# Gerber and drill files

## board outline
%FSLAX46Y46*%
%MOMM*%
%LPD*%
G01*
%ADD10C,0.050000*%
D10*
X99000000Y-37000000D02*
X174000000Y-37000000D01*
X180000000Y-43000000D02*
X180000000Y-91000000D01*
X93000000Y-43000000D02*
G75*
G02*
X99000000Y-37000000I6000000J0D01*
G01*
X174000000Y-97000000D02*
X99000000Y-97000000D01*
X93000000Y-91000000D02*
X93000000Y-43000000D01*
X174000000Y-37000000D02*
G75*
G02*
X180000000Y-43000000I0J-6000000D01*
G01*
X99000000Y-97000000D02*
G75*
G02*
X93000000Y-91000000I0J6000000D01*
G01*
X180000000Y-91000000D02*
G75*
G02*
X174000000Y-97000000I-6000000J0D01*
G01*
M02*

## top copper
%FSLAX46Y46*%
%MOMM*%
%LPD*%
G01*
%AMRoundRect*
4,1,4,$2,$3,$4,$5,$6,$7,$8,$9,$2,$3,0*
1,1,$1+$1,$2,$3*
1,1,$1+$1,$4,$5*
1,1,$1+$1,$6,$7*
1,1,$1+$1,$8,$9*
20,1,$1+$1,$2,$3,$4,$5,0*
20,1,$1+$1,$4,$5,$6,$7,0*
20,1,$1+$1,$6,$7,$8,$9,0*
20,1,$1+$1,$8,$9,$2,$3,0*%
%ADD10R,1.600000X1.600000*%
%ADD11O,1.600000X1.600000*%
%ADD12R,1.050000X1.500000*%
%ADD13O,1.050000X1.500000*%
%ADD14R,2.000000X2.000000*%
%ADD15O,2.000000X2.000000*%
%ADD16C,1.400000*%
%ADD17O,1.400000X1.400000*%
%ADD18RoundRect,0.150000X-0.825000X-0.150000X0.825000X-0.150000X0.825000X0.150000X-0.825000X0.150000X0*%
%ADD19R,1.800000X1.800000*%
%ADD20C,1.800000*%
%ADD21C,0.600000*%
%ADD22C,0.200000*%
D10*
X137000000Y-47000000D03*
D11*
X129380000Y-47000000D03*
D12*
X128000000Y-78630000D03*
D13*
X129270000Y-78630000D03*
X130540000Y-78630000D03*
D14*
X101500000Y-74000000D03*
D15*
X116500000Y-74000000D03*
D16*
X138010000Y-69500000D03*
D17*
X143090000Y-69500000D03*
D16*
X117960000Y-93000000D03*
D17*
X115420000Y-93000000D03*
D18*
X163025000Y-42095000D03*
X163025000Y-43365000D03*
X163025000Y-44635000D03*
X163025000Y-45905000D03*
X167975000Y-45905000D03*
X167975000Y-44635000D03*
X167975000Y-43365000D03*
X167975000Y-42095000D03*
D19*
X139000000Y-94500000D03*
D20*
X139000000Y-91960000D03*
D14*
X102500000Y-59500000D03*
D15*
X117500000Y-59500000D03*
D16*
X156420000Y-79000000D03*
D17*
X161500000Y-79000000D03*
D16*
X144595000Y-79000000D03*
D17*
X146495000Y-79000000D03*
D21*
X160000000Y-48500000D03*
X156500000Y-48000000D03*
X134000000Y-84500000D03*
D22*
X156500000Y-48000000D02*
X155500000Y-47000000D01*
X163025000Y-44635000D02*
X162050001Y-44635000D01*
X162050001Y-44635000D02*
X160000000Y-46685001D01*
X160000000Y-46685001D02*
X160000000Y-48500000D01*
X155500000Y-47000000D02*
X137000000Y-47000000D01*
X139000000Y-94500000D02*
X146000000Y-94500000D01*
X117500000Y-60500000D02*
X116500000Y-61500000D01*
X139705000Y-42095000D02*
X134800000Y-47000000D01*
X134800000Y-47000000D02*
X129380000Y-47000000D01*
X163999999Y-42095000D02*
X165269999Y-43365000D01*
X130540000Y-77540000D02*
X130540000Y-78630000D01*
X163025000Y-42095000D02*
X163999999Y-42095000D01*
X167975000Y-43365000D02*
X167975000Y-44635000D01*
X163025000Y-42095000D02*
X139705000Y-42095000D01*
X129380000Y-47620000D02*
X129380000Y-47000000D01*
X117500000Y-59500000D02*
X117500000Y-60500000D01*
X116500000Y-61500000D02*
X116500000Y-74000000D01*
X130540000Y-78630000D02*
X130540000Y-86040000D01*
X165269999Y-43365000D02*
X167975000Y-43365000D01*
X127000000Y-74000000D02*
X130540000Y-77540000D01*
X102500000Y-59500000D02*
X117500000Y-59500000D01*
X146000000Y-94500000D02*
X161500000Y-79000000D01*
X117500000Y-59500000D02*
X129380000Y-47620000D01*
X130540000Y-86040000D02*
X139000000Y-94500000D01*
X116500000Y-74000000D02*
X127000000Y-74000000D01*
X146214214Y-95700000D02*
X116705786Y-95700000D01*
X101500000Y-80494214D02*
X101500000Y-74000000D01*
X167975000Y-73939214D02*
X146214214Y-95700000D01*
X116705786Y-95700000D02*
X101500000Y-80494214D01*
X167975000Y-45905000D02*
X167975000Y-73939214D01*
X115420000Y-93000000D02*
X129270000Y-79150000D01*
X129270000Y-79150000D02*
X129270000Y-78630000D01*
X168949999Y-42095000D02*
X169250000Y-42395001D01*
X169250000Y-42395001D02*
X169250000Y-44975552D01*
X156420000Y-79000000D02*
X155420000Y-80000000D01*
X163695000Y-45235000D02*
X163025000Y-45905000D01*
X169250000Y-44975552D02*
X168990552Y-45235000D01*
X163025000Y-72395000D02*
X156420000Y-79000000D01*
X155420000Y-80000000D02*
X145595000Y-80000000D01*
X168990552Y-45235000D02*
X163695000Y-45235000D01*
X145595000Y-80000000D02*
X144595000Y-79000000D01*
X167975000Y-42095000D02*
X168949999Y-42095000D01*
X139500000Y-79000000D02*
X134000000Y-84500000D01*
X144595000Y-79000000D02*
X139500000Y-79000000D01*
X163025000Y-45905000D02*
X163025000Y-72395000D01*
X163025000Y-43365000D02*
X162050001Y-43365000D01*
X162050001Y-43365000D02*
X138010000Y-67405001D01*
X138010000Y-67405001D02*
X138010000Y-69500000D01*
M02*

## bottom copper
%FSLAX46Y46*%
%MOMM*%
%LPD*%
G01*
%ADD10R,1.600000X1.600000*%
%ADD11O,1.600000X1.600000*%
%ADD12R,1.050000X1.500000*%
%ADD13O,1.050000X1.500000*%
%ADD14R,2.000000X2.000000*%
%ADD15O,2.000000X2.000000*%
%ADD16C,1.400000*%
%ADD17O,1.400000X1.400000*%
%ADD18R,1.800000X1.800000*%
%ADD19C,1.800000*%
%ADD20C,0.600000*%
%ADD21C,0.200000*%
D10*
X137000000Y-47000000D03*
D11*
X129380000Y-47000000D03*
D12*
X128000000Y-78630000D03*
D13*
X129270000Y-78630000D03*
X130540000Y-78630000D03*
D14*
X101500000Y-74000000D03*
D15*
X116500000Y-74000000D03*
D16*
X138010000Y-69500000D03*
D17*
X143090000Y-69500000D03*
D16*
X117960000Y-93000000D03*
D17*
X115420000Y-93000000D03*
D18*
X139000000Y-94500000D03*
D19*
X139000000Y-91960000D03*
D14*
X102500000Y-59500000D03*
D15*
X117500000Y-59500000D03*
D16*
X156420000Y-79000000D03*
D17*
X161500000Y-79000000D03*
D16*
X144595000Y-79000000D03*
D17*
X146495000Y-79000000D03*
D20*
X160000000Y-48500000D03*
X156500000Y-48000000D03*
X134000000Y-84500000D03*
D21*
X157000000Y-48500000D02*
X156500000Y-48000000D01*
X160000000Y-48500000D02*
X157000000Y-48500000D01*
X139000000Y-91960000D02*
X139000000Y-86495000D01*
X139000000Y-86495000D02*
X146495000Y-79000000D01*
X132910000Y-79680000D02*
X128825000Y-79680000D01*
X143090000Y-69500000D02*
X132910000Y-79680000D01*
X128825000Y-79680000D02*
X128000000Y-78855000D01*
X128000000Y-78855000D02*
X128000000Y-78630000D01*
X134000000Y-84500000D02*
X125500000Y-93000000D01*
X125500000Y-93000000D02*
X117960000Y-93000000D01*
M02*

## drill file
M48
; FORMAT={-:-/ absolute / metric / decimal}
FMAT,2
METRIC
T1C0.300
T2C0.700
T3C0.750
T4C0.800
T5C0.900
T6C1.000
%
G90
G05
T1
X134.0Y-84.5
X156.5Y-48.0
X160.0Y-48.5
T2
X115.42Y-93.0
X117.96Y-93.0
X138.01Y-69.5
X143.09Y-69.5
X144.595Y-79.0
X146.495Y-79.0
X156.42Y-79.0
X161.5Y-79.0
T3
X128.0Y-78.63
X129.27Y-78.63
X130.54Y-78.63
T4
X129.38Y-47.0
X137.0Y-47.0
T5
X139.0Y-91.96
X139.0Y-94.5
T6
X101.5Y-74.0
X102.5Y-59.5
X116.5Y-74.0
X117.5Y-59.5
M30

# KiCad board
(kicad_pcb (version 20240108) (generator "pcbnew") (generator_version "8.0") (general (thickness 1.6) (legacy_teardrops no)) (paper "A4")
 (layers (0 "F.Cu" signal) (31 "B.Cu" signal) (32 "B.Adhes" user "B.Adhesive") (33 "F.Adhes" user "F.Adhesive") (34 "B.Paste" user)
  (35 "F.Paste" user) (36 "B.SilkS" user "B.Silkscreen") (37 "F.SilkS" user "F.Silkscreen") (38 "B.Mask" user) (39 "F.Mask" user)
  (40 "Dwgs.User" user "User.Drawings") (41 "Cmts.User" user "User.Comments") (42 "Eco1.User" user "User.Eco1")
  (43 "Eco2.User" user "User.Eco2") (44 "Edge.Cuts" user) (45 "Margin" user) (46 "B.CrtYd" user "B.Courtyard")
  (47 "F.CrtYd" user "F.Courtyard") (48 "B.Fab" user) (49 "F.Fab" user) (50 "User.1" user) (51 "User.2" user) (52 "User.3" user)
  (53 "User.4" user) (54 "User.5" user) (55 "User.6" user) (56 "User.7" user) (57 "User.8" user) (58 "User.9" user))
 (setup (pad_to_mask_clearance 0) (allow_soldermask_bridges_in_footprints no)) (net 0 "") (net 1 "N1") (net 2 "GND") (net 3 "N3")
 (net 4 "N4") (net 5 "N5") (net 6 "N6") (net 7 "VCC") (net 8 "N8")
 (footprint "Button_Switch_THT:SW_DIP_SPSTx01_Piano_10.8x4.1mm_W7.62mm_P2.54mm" (layer "F.Cu") (at 137 47 180)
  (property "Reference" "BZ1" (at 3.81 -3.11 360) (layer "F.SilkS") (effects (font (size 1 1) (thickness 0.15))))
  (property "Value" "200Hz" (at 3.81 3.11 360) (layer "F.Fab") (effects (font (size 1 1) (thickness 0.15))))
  (pad "1" thru_hole rect (at 0 0 180) (size 1.6 1.6) (drill 0.8) (layers "*.Cu" "*.Mask") (remove_unused_layers no) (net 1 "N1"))
  (pad "2" thru_hole oval (at 7.62 0 180) (size 1.6 1.6) (drill 0.8) (layers "*.Cu" "*.Mask") (remove_unused_layers no) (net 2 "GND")))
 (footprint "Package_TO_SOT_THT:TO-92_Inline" (layer "F.Cu") (at 128 78.63)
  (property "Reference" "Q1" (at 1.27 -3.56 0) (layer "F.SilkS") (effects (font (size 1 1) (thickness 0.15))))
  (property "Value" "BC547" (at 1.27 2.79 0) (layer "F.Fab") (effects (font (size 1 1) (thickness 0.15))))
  (pad "1" thru_hole rect (at 0 0) (size 1.05 1.5) (drill 0.75) (layers "*.Cu" "*.Mask") (remove_unused_layers no) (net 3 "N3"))
  (pad "2" thru_hole oval (at 1.27 0) (size 1.05 1.5) (drill 0.75) (layers "*.Cu" "*.Mask") (remove_unused_layers no) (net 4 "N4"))
  (pad "3" thru_hole oval (at 2.54 0) (size 1.05 1.5) (drill 0.75) (layers "*.Cu" "*.Mask") (remove_unused_layers no) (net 2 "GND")))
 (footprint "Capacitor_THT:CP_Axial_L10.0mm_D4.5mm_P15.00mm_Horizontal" (layer "F.Cu") (at 101.5 74)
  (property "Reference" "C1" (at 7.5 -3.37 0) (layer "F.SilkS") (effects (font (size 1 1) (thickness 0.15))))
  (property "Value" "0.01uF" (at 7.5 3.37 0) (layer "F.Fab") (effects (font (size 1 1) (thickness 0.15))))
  (pad "1" thru_hole rect (at 0 0) (size 2 2) (drill 1) (layers "*.Cu" "*.Mask") (remove_unused_layers no) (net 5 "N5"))
  (pad "2" thru_hole oval (at 15 0) (size 2 2) (drill 1) (layers "*.Cu" "*.Mask") (remove_unused_layers no) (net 2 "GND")))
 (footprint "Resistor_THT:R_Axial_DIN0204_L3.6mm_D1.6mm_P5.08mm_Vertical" (layer "F.Cu") (at 138.01 69.5)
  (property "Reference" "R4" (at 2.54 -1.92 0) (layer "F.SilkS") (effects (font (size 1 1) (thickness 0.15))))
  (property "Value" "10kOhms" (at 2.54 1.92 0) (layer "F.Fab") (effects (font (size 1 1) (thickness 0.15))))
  (pad "1" thru_hole circle (at 0 0) (size 1.4 1.4) (drill 0.7) (layers "*.Cu" "*.Mask") (remove_unused_layers no) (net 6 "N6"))
  (pad "2" thru_hole oval (at 5.08 0) (size 1.4 1.4) (drill 0.7) (layers "*.Cu" "*.Mask") (remove_unused_layers no) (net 3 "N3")))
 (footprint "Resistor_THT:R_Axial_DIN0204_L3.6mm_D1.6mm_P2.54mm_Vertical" (layer "F.Cu") (at 117.96 93 180)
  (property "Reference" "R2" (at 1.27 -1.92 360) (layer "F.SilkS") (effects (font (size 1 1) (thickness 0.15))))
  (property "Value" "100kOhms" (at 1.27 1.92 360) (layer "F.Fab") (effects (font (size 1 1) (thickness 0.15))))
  (pad "1" thru_hole circle (at 0 0 180) (size 1.4 1.4) (drill 0.7) (layers "*.Cu" "*.Mask") (remove_unused_layers no) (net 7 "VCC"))
  (pad "2" thru_hole oval (at 2.54 0 180) (size 1.4 1.4) (drill 0.7) (layers "*.Cu" "*.Mask") (remove_unused_layers no) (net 4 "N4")))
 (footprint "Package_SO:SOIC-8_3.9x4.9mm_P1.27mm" (layer "F.Cu") (at 165.5 44)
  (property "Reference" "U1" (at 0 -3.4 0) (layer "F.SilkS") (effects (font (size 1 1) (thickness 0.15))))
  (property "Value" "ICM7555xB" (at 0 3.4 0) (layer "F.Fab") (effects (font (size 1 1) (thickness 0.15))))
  (pad "1" smd roundrect (at -2.475 -1.905) (size 1.95 0.6) (layers "F.Cu" "F.Paste" "F.Mask") (roundrect_rratio 0.25) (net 2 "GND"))
  (pad "2" smd roundrect (at -2.475 -0.635) (size 1.95 0.6) (layers "F.Cu" "F.Paste" "F.Mask") (roundrect_rratio 0.25) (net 6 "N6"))
  (pad "3" smd roundrect (at -2.475 0.635) (size 1.95 0.6) (layers "F.Cu" "F.Paste" "F.Mask") (roundrect_rratio 0.25) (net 1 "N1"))
  (pad "4" smd roundrect (at -2.475 1.905) (size 1.95 0.6) (layers "F.Cu" "F.Paste" "F.Mask") (roundrect_rratio 0.25) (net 7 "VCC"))
  (pad "5" smd roundrect (at 2.475 1.905) (size 1.95 0.6) (layers "F.Cu" "F.Paste" "F.Mask") (roundrect_rratio 0.25) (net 5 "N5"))
  (pad "6" smd roundrect (at 2.475 0.635) (size 1.95 0.6) (layers "F.Cu" "F.Paste" "F.Mask") (roundrect_rratio 0.25) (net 2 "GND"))
  (pad "7" smd roundrect (at 2.475 -0.635) (size 1.95 0.6) (layers "F.Cu" "F.Paste" "F.Mask") (roundrect_rratio 0.25) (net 2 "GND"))
  (pad "8" smd roundrect (at 2.475 -1.905) (size 1.95 0.6) (layers "F.Cu" "F.Paste" "F.Mask") (roundrect_rratio 0.25) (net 7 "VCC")))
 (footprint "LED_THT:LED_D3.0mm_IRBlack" (layer "F.Cu") (at 139 94.5 90)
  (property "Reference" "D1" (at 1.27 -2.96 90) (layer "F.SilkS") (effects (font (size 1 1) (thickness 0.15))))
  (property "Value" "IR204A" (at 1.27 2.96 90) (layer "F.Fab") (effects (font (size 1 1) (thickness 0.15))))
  (pad "1" thru_hole rect (at 0 0 90) (size 1.8 1.8) (drill 0.9) (layers "*.Cu" "*.Mask") (remove_unused_layers no) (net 2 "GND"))
  (pad "2" thru_hole circle (at 2.54 0 90) (size 1.8 1.8) (drill 0.9) (layers "*.Cu" "*.Mask") (remove_unused_layers no) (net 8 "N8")))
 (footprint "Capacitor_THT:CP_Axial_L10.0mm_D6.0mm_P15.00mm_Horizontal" (layer "F.Cu") (at 102.5 59.5)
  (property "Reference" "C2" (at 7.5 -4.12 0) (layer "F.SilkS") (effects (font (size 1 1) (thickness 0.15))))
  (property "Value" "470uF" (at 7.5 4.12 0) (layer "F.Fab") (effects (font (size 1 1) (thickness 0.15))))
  (pad "1" thru_hole rect (at 0 0) (size 2 2) (drill 1) (layers "*.Cu" "*.Mask") (remove_unused_layers no) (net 2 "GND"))
  (pad "2" thru_hole oval (at 15 0) (size 2 2) (drill 1) (layers "*.Cu" "*.Mask") (remove_unused_layers no) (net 2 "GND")))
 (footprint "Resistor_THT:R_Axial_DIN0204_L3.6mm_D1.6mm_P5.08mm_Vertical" (layer "F.Cu") (at 156.42 79)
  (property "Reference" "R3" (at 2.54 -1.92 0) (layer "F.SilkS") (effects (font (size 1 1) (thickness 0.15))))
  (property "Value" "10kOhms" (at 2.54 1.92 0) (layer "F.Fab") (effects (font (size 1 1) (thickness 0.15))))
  (pad "1" thru_hole circle (at 0 0) (size 1.4 1.4) (drill 0.7) (layers "*.Cu" "*.Mask") (remove_unused_layers no) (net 7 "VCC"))
  (pad "2" thru_hole oval (at 5.08 0) (size 1.4 1.4) (drill 0.7) (layers "*.Cu" "*.Mask") (remove_unused_layers no) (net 2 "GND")))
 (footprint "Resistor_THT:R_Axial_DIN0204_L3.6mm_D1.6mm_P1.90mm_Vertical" (layer "F.Cu") (at 144.595 79)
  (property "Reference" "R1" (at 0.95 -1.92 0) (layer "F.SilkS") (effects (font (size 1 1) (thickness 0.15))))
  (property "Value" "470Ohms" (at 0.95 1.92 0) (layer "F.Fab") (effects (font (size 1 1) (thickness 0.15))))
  (pad "1" thru_hole circle (at 0 0) (size 1.4 1.4) (drill 0.7) (layers "*.Cu" "*.Mask") (remove_unused_layers no) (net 7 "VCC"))
  (pad "2" thru_hole oval (at 1.9 0) (size 1.4 1.4) (drill 0.7) (layers "*.Cu" "*.Mask") (remove_unused_layers no) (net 8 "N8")))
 (gr_line (start 99 37) (end 174 37) (stroke (width 0.05) (type default)) (layer "Edge.Cuts"))
 (gr_line (start 180 43) (end 180 91) (stroke (width 0.05) (type default)) (layer "Edge.Cuts"))
 (gr_arc (start 93 43) (mid 94.757359 38.757359) (end 99 37) (stroke (width 0.05) (type default)) (layer "Edge.Cuts"))
 (gr_line (start 174 97) (end 99 97) (stroke (width 0.05) (type default)) (layer "Edge.Cuts"))
 (gr_line (start 93 91) (end 93 43) (stroke (width 0.05) (type default)) (layer "Edge.Cuts"))
 (gr_arc (start 174 37) (mid 178.242641 38.757359) (end 180 43) (stroke (width 0.05) (type default)) (layer "Edge.Cuts"))
 (gr_arc (start 99 97) (mid 94.757359 95.242641) (end 93 91) (stroke (width 0.05) (type default)) (layer "Edge.Cuts"))
 (gr_arc (start 180 91) (mid 178.242641 95.242641) (end 174 97) (stroke (width 0.05) (type default)) (layer "Edge.Cuts"))
 (segment (start 156.5 48) (end 155.5 47) (width 0.2) (layer "F.Cu") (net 1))
 (segment (start 163.025 44.635) (end 162.050001 44.635) (width 0.2) (layer "F.Cu") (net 1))
 (segment (start 162.050001 44.635) (end 160 46.685001) (width 0.2) (layer "F.Cu") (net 1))
 (segment (start 160 46.685001) (end 160 48.5) (width 0.2) (layer "F.Cu") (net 1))
 (segment (start 155.5 47) (end 137 47) (width 0.2) (layer "F.Cu") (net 1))
 (via (at 160 48.5) (size 0.6) (drill 0.3) (layers "F.Cu" "B.Cu") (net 1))
 (via (at 156.5 48) (size 0.6) (drill 0.3) (layers "F.Cu" "B.Cu") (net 1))
 (segment (start 157 48.5) (end 156.5 48) (width 0.2) (layer "B.Cu") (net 1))
 (segment (start 160 48.5) (end 157 48.5) (width 0.2) (layer "B.Cu") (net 1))
 (segment (start 139 94.5) (end 146 94.5) (width 0.2) (layer "F.Cu") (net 2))
 (segment (start 117.5 60.5) (end 116.5 61.5) (width 0.2) (layer "F.Cu") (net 2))
 (segment (start 139.705 42.095) (end 134.8 47) (width 0.2) (layer "F.Cu") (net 2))
 (segment (start 134.8 47) (end 129.38 47) (width 0.2) (layer "F.Cu") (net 2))
 (segment (start 163.999999 42.095) (end 165.269999 43.365) (width 0.2) (layer "F.Cu") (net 2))
 (segment (start 130.54 77.54) (end 130.54 78.63) (width 0.2) (layer "F.Cu") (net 2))
 (segment (start 163.025 42.095) (end 163.999999 42.095) (width 0.2) (layer "F.Cu") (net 2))
 (segment (start 167.975 43.365) (end 167.975 44.635) (width 0.2) (layer "F.Cu") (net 2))
 (segment (start 163.025 42.095) (end 139.705 42.095) (width 0.2) (layer "F.Cu") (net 2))
 (segment (start 129.38 47.62) (end 129.38 47) (width 0.2) (layer "F.Cu") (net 2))
 (segment (start 117.5 59.5) (end 117.5 60.5) (width 0.2) (layer "F.Cu") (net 2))
 (segment (start 116.5 61.5) (end 116.5 74) (width 0.2) (layer "F.Cu") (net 2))
 (segment (start 130.54 78.63) (end 130.54 86.04) (width 0.2) (layer "F.Cu") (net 2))
 (segment (start 165.269999 43.365) (end 167.975 43.365) (width 0.2) (layer "F.Cu") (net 2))
 (segment (start 127 74) (end 130.54 77.54) (width 0.2) (layer "F.Cu") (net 2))
 (segment (start 102.5 59.5) (end 117.5 59.5) (width 0.2) (layer "F.Cu") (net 2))
 (segment (start 146 94.5) (end 161.5 79) (width 0.2) (layer "F.Cu") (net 2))
 (segment (start 117.5 59.5) (end 129.38 47.62) (width 0.2) (layer "F.Cu") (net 2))
 (segment (start 130.54 86.04) (end 139 94.5) (width 0.2) (layer "F.Cu") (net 2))
 (segment (start 116.5 74) (end 127 74) (width 0.2) (layer "F.Cu") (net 2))
 (segment (start 146.214214 95.7) (end 116.705786 95.7) (width 0.2) (layer "F.Cu") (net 5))
 (segment (start 101.5 80.494214) (end 101.5 74) (width 0.2) (layer "F.Cu") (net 5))
 (segment (start 167.975 73.939214) (end 146.214214 95.7) (width 0.2) (layer "F.Cu") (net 5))
 (segment (start 116.705786 95.7) (end 101.5 80.494214) (width 0.2) (layer "F.Cu") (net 5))
 (segment (start 167.975 45.905) (end 167.975 73.939214) (width 0.2) (layer "F.Cu") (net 5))
 (segment (start 139 91.96) (end 139 86.495) (width 0.2) (layer "B.Cu") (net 8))
 (segment (start 139 86.495) (end 146.495 79) (width 0.2) (layer "B.Cu") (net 8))
 (segment (start 115.42 93) (end 129.27 79.15) (width 0.2) (layer "F.Cu") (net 4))
 (segment (start 129.27 79.15) (end 129.27 78.63) (width 0.2) (layer "F.Cu") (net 4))
 (segment (start 132.91 79.68) (end 128.825 79.68) (width 0.2) (layer "B.Cu") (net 3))
 (segment (start 143.09 69.5) (end 132.91 79.68) (width 0.2) (layer "B.Cu") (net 3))
 (segment (start 128.825 79.68) (end 128 78.855) (width 0.2) (layer "B.Cu") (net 3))
 (segment (start 128 78.855) (end 128 78.63) (width 0.2) (layer "B.Cu") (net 3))
 (segment (start 168.949999 42.095) (end 169.25 42.395001) (width 0.2) (layer "F.Cu") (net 7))
 (segment (start 169.25 42.395001) (end 169.25 44.975552) (width 0.2) (layer "F.Cu") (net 7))
 (segment (start 156.42 79) (end 155.42 80) (width 0.2) (layer "F.Cu") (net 7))
 (segment (start 163.695 45.235) (end 163.025 45.905) (width 0.2) (layer "F.Cu") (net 7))
 (segment (start 169.25 44.975552) (end 168.990552 45.235) (width 0.2) (layer "F.Cu") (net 7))
 (segment (start 163.025 72.395) (end 156.42 79) (width 0.2) (layer "F.Cu") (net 7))
 (segment (start 155.42 80) (end 145.595 80) (width 0.2) (layer "F.Cu") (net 7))
 (segment (start 168.990552 45.235) (end 163.695 45.235) (width 0.2) (layer "F.Cu") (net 7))
 (segment (start 145.595 80) (end 144.595 79) (width 0.2) (layer "F.Cu") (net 7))
 (segment (start 167.975 42.095) (end 168.949999 42.095) (width 0.2) (layer "F.Cu") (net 7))
 (segment (start 139.5 79) (end 134 84.5) (width 0.2) (layer "F.Cu") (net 7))
 (segment (start 144.595 79) (end 139.5 79) (width 0.2) (layer "F.Cu") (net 7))
 (segment (start 163.025 45.905) (end 163.025 72.395) (width 0.2) (layer "F.Cu") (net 7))
 (via (at 134 84.5) (size 0.6) (drill 0.3) (layers "F.Cu" "B.Cu") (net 7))
 (segment (start 134 84.5) (end 125.5 93) (width 0.2) (layer "B.Cu") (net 7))
 (segment (start 125.5 93) (end 117.96 93) (width 0.2) (layer "B.Cu") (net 7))
 (segment (start 163.025 43.365) (end 162.050001 43.365) (width 0.2) (layer "F.Cu") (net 6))
 (segment (start 162.050001 43.365) (end 138.01 67.405001) (width 0.2) (layer "F.Cu") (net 6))
 (segment (start 138.01 67.405001) (end 138.01 69.5) (width 0.2) (layer "F.Cu") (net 6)))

